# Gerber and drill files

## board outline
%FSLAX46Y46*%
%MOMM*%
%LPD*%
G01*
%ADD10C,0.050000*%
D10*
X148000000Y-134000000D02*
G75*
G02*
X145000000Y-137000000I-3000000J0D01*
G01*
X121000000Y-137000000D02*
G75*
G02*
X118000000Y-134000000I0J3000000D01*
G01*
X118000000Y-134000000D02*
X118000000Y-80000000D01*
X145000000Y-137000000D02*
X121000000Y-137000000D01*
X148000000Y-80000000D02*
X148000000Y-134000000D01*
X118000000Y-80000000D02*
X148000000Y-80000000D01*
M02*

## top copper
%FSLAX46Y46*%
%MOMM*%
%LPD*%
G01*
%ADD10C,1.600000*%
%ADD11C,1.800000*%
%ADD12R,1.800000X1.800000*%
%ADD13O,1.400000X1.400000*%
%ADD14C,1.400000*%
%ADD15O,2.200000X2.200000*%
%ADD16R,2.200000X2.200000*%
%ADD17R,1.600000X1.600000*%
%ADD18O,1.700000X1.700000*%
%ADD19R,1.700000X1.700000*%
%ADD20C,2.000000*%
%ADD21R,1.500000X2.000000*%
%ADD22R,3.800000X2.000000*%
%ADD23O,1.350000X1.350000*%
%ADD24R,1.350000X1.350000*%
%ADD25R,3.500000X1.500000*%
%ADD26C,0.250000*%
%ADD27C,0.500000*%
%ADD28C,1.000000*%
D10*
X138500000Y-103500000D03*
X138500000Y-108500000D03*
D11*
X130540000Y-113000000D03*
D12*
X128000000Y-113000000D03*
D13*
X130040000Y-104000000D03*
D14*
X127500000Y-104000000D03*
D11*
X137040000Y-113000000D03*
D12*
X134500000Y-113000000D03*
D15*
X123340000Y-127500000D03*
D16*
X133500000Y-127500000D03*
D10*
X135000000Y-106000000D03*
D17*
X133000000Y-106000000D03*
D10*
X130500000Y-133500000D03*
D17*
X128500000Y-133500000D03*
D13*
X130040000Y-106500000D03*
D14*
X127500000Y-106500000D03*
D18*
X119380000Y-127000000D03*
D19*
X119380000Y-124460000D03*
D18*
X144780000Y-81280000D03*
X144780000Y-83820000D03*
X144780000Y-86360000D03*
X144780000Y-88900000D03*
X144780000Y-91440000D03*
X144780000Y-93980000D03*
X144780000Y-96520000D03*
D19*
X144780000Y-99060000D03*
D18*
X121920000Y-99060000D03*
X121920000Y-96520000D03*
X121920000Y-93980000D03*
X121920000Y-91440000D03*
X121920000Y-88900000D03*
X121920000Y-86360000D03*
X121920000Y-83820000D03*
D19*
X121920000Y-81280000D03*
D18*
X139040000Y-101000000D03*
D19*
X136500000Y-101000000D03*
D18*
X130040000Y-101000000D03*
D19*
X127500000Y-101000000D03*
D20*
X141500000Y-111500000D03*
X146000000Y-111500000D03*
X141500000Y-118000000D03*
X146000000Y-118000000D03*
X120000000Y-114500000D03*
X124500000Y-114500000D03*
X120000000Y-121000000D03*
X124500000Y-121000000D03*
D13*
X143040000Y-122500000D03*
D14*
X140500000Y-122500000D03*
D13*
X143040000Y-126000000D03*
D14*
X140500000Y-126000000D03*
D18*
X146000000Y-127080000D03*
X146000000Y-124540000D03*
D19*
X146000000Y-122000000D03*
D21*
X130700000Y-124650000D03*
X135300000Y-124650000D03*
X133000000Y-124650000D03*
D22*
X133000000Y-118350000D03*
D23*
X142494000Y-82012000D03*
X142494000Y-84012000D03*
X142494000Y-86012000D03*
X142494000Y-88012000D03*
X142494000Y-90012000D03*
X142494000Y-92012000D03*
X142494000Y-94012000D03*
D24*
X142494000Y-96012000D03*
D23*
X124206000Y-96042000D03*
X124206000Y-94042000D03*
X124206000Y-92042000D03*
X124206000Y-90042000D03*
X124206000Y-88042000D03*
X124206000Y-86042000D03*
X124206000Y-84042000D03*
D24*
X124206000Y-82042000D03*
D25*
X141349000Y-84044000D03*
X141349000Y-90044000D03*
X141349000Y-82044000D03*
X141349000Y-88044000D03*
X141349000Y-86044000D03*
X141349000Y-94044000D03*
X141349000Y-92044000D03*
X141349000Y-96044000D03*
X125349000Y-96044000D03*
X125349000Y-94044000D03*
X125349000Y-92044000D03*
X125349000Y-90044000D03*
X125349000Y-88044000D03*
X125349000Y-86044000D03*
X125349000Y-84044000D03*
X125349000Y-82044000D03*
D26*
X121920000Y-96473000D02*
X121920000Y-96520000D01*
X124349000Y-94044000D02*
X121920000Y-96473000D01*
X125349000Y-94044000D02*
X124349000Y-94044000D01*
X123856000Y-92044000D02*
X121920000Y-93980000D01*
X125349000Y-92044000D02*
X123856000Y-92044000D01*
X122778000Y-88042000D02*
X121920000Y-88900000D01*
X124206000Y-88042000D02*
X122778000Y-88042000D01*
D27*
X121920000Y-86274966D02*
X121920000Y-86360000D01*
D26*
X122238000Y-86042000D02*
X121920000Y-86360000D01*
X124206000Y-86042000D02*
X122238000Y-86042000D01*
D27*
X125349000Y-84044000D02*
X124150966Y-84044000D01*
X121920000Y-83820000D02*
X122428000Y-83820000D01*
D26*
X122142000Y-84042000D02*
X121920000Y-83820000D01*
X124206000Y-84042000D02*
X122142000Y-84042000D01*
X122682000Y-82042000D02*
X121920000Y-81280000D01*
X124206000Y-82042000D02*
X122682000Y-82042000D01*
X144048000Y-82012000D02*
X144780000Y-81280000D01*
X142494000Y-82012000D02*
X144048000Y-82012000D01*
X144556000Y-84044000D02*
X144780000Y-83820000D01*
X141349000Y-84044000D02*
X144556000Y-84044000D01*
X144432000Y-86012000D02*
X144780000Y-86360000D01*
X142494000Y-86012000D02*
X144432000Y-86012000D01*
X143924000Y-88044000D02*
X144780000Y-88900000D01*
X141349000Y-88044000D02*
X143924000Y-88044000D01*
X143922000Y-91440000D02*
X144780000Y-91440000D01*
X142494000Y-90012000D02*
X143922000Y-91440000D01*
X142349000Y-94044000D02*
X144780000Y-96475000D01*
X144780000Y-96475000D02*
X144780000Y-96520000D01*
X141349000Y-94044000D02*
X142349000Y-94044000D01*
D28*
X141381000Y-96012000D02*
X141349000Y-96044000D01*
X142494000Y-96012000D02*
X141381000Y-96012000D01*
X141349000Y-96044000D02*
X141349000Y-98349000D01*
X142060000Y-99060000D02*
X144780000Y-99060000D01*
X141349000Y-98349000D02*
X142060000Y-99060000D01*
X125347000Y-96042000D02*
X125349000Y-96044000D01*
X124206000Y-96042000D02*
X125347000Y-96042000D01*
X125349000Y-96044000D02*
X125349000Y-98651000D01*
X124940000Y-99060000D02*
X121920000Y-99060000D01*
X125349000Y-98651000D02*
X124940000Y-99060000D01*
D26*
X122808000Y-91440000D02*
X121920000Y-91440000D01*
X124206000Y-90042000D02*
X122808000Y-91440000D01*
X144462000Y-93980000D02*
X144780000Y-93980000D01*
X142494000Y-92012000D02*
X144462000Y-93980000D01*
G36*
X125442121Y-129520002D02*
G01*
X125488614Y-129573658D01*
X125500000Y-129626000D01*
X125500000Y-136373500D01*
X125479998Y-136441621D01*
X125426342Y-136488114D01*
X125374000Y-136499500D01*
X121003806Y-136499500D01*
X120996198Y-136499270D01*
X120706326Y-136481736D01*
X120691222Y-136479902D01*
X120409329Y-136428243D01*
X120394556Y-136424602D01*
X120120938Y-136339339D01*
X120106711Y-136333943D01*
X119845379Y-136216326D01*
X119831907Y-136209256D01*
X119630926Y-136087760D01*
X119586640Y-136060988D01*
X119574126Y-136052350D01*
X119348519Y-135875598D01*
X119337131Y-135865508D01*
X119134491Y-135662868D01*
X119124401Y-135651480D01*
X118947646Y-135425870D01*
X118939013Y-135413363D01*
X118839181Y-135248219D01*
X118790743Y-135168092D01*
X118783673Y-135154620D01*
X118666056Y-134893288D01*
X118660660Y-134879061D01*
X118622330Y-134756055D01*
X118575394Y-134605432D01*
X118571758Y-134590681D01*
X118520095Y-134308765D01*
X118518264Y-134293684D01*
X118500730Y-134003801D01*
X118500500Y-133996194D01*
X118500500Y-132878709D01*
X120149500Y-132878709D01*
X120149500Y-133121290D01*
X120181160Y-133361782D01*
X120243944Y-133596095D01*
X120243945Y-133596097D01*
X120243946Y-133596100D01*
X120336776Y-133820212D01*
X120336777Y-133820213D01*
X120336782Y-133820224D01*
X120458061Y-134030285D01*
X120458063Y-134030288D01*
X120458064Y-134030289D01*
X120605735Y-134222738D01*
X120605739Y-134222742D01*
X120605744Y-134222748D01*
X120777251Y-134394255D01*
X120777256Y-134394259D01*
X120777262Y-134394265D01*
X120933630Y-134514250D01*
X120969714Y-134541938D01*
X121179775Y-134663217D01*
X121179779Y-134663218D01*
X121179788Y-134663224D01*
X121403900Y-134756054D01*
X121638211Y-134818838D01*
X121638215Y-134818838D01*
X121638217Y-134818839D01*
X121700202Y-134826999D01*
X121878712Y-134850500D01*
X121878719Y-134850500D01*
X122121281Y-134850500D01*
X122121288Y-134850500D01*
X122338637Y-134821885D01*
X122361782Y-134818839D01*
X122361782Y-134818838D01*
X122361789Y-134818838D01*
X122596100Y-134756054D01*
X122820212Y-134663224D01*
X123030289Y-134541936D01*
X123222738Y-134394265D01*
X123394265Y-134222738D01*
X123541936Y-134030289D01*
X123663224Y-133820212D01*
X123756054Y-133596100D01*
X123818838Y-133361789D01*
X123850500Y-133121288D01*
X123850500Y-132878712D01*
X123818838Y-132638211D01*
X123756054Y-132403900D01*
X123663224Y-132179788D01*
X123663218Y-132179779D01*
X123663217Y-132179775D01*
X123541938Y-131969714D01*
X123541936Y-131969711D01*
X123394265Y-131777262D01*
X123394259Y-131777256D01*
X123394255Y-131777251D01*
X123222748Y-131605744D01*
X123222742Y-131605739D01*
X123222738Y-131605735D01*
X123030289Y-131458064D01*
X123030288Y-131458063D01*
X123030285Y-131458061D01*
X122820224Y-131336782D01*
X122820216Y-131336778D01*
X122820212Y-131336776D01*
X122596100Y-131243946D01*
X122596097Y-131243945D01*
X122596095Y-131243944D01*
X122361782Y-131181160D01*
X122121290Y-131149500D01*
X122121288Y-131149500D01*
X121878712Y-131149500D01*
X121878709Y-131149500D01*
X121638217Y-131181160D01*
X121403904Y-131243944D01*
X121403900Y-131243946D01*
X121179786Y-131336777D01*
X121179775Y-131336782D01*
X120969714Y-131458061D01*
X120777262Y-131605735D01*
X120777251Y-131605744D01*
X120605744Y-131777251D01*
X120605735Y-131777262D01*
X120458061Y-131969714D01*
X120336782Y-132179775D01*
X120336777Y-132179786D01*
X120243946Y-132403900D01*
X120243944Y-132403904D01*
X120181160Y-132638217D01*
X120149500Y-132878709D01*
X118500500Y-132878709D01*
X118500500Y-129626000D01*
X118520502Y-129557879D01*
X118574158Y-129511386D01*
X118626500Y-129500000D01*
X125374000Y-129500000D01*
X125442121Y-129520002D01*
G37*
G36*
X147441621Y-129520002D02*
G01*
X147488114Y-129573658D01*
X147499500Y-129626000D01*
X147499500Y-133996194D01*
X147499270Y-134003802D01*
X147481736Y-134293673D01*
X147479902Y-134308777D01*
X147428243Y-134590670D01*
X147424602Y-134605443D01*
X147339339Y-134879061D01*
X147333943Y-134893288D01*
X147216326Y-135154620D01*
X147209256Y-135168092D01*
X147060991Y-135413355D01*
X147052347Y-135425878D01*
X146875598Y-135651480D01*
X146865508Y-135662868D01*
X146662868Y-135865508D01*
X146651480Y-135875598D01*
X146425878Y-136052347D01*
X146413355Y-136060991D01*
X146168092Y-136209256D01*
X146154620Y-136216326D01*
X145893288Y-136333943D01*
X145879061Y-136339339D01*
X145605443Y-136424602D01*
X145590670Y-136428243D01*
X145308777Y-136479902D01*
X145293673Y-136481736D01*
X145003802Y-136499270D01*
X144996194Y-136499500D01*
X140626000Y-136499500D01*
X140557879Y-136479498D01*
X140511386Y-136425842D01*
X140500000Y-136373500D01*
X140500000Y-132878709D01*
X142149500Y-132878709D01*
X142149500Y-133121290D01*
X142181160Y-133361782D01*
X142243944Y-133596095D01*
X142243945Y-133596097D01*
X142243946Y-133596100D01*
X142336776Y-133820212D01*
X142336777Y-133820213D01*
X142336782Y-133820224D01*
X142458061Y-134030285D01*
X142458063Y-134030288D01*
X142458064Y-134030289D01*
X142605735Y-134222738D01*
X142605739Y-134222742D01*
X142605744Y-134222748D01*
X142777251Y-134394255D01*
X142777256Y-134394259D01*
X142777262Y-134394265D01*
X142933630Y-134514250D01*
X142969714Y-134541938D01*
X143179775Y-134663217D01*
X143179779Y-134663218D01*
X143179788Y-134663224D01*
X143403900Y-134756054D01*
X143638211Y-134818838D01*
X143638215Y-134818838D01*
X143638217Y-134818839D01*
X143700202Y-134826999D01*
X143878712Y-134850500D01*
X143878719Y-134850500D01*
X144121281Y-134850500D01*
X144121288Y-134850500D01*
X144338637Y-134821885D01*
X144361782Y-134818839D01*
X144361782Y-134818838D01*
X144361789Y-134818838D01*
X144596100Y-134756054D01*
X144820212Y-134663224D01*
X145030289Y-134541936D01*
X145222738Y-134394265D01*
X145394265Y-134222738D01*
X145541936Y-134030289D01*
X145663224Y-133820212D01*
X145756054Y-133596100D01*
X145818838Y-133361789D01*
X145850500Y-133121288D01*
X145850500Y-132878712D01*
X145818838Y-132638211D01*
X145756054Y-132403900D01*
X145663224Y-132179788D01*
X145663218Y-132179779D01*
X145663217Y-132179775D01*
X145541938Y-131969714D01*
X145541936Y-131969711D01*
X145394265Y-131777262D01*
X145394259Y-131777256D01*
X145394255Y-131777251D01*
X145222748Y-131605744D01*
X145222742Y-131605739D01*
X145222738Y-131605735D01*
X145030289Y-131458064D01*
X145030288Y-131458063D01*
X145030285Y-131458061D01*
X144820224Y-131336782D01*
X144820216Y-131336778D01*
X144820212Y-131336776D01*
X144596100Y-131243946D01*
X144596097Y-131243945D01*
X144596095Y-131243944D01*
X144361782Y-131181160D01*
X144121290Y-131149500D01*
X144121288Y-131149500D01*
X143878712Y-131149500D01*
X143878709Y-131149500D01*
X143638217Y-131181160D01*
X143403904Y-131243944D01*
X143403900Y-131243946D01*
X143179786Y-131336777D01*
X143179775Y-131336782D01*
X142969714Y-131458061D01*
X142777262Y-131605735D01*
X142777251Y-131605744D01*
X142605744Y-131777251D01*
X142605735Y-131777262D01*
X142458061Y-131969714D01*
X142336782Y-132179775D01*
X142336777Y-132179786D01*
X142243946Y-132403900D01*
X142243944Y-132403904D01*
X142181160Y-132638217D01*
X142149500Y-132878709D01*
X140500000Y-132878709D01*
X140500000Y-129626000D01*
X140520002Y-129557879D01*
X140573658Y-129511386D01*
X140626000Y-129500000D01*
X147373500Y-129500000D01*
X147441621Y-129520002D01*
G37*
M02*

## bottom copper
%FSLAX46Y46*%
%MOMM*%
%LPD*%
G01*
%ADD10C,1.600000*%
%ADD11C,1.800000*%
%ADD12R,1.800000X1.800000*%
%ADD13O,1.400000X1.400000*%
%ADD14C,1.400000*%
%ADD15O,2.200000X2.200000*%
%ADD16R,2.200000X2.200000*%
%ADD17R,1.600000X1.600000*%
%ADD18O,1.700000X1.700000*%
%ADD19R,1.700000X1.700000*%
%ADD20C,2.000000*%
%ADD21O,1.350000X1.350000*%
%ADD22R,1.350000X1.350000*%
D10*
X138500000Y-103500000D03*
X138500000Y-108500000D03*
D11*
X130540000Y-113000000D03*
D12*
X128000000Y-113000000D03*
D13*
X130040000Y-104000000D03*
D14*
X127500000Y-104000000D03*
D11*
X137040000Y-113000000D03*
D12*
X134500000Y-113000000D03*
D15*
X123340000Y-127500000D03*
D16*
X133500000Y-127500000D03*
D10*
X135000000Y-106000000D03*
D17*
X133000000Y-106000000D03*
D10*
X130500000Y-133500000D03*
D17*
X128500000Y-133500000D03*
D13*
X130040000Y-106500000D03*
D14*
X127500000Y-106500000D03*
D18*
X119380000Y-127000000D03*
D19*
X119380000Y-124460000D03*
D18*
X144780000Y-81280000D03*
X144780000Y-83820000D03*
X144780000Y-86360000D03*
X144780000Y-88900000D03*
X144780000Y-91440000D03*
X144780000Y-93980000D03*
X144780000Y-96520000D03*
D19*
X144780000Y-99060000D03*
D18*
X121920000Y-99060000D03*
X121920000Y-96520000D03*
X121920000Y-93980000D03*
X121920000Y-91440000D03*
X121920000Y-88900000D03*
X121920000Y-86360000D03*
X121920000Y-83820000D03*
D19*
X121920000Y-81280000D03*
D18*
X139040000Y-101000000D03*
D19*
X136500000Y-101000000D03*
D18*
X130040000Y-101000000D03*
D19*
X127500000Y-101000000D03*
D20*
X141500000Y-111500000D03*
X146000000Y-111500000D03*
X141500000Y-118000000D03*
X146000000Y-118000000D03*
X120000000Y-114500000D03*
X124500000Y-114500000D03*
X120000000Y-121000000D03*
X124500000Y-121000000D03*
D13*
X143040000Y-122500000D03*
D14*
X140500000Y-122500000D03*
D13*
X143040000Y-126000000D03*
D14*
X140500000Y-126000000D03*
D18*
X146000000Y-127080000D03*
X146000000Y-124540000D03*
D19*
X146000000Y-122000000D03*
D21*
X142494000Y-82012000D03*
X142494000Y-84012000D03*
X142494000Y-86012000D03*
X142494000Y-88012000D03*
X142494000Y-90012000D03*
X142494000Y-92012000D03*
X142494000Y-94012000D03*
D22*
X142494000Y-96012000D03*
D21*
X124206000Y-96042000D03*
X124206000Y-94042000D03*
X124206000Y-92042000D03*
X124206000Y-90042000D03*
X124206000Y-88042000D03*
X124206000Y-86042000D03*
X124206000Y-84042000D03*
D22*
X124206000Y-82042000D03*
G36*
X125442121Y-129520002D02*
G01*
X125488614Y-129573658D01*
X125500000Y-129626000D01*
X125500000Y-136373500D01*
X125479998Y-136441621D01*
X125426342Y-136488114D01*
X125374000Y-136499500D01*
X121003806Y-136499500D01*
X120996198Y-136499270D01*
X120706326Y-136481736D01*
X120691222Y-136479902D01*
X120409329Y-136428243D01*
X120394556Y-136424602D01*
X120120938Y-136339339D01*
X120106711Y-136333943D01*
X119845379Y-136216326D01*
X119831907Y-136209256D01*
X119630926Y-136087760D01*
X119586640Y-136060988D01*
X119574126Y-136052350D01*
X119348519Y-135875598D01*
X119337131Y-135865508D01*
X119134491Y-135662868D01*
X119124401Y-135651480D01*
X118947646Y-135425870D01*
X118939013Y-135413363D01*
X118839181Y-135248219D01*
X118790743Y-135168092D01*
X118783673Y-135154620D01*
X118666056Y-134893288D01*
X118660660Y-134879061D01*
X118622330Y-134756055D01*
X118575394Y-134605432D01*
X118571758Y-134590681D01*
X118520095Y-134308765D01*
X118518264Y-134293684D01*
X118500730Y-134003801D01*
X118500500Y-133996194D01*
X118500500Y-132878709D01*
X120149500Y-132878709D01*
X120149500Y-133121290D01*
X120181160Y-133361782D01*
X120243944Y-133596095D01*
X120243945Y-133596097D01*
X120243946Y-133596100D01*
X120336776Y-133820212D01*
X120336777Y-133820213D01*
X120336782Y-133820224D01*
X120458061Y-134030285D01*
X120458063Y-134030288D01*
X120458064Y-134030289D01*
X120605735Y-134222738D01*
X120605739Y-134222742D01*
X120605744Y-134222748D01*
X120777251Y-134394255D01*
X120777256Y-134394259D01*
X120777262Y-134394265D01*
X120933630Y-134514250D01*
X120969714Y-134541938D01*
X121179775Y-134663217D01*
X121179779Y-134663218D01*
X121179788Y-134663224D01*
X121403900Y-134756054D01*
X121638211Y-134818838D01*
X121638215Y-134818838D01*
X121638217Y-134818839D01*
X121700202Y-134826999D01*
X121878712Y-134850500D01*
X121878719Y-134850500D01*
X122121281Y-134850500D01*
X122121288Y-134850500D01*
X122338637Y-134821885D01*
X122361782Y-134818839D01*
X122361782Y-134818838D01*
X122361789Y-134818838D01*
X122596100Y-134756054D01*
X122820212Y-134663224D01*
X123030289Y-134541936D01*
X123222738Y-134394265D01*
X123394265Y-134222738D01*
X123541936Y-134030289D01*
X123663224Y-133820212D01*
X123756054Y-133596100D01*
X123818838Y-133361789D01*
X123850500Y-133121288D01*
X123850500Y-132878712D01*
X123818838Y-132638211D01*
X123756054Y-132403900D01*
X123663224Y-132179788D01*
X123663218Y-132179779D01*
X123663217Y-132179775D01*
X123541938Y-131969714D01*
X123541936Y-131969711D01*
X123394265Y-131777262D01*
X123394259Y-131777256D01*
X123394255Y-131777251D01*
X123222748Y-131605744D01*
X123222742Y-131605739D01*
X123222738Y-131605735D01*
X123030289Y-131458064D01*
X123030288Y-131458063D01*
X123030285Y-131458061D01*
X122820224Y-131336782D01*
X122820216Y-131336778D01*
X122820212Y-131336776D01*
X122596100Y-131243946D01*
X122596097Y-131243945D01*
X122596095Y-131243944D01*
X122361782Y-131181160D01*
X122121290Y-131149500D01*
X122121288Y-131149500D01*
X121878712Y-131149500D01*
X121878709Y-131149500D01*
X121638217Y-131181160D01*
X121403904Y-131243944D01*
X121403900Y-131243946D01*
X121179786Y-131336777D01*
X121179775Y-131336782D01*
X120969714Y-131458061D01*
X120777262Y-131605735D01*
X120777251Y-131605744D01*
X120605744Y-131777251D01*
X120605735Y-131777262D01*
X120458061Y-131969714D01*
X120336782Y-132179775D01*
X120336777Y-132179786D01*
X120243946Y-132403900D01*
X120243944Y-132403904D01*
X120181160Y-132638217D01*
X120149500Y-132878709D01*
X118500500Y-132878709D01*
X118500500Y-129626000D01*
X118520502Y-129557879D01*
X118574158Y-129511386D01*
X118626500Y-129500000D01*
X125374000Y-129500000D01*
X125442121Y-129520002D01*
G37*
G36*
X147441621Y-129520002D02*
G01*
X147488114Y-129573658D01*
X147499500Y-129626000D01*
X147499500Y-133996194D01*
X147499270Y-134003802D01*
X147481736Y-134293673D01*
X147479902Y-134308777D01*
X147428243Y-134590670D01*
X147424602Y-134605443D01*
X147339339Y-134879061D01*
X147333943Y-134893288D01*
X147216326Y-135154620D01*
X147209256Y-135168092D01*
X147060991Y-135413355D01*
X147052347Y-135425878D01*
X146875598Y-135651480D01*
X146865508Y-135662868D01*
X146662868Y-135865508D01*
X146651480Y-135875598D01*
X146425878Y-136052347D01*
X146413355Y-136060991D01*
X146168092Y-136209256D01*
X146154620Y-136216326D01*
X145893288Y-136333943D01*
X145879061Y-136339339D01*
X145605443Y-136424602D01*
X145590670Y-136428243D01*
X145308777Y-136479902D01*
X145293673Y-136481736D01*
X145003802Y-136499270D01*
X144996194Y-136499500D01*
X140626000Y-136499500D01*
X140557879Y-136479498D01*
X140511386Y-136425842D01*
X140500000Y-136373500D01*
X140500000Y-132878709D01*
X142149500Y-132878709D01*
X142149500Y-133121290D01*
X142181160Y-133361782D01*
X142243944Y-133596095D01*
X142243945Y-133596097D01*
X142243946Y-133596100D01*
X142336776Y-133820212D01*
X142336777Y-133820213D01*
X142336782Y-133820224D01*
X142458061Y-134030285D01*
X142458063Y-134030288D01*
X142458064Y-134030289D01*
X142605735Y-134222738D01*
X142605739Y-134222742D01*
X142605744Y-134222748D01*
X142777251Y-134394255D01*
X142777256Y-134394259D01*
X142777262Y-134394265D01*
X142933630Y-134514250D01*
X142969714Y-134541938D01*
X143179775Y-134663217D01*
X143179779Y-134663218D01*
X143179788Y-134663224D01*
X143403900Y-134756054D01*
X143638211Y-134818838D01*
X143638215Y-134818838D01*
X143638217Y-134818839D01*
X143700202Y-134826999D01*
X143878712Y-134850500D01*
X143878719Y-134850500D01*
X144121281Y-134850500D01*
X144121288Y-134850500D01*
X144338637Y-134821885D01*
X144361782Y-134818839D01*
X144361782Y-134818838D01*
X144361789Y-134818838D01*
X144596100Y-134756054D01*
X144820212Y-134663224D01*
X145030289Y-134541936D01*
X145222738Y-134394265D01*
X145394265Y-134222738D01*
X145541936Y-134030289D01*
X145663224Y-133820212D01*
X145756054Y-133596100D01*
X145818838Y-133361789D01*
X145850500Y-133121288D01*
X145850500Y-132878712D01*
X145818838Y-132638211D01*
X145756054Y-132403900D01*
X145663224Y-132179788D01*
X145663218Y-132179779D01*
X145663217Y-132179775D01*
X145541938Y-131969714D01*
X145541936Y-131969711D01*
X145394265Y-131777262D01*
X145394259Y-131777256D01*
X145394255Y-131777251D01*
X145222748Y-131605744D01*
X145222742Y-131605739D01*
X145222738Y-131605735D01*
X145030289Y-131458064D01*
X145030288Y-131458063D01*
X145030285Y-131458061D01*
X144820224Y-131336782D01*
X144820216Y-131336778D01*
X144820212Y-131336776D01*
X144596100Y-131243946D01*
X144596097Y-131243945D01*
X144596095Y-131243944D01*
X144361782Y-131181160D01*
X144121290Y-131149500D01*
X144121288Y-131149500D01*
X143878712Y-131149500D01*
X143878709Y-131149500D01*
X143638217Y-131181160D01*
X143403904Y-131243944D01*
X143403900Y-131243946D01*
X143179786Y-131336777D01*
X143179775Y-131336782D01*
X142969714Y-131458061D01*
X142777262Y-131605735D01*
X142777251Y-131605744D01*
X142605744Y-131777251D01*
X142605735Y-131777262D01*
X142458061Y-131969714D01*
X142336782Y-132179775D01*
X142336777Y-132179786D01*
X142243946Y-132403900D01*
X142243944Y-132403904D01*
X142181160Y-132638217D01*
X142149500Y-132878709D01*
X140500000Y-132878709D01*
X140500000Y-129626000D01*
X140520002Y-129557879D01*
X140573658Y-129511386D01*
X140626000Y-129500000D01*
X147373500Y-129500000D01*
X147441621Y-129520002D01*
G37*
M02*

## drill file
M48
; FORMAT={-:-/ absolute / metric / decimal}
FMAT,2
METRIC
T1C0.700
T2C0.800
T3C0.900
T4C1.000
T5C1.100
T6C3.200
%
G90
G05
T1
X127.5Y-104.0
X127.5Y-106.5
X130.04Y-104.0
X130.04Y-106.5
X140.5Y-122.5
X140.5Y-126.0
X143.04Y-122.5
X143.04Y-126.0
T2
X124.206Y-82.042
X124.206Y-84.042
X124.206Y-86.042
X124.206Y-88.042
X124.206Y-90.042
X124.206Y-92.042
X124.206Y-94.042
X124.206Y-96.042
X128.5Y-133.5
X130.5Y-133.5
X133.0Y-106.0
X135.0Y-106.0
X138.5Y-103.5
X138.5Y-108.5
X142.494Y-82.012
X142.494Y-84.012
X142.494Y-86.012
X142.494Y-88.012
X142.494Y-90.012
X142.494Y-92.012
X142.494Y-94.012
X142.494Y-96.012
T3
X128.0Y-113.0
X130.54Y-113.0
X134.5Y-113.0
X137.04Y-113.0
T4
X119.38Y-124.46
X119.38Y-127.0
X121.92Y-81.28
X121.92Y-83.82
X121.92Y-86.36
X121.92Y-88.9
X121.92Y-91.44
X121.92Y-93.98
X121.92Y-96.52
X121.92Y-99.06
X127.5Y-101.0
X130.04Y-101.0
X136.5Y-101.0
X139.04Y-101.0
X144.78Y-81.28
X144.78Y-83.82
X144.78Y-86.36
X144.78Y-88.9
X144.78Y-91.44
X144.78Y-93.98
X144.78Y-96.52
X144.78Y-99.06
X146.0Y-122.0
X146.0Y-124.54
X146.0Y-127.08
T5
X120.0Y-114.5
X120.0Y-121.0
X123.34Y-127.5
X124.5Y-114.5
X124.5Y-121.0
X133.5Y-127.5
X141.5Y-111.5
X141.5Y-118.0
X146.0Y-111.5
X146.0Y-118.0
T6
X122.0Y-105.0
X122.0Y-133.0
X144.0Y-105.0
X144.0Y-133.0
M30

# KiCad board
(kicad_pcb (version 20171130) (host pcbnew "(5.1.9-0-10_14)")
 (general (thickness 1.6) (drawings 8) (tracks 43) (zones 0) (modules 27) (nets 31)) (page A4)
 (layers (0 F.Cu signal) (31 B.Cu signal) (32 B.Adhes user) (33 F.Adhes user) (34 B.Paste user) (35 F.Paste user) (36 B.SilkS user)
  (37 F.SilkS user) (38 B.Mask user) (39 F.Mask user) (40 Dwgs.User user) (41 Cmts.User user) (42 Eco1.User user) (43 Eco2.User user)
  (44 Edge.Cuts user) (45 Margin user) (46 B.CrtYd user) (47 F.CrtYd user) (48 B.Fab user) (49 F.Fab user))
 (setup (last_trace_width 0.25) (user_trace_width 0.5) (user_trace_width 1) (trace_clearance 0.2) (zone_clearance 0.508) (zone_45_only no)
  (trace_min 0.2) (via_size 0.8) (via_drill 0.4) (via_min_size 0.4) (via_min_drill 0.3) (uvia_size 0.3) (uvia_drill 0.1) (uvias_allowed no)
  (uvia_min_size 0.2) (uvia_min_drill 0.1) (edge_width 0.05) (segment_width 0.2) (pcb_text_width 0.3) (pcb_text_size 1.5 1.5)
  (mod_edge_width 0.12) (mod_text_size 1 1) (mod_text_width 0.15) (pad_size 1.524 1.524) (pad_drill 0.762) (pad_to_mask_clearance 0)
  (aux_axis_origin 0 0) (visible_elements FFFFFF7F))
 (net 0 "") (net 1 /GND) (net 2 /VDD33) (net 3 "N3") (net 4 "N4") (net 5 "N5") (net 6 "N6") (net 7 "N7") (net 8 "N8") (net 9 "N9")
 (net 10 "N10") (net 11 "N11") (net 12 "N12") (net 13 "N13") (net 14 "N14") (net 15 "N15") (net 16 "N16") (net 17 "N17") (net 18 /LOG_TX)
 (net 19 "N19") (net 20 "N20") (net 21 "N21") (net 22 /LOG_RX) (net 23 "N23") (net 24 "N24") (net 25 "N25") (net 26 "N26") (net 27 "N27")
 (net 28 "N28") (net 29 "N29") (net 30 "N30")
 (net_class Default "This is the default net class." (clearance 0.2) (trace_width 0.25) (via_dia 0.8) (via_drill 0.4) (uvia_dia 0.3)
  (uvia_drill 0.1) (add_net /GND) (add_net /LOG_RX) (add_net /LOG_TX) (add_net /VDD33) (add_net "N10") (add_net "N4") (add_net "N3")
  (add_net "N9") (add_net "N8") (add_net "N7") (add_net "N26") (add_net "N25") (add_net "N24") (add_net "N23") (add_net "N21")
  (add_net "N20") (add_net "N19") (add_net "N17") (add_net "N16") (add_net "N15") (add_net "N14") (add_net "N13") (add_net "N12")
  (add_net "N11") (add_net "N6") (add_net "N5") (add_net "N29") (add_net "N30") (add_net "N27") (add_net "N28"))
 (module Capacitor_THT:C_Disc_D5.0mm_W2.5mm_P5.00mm (layer F.Cu) (at 138.5 108.5 90)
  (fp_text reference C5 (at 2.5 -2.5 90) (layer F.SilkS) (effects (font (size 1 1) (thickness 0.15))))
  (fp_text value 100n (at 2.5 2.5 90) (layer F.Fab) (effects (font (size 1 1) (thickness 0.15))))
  (pad 2 thru_hole circle (at 5 0 90) (size 1.6 1.6) (drill 0.8) (layers *.Cu *.Mask) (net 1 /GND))
  (pad 1 thru_hole circle (at 0 0 90) (size 1.6 1.6) (drill 0.8) (layers *.Cu *.Mask) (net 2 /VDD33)))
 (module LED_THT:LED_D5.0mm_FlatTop (layer F.Cu) (at 128 113)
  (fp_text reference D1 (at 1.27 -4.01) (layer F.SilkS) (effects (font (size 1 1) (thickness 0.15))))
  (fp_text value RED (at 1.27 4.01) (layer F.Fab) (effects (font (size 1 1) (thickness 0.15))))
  (pad 2 thru_hole circle (at 2.54 0) (size 1.8 1.8) (drill 0.9) (layers *.Cu *.Mask) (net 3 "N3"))
  (pad 1 thru_hole rect (at 0 0) (size 1.8 1.8) (drill 0.9) (layers *.Cu *.Mask) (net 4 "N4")))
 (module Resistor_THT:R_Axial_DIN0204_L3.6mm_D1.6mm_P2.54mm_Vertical (layer F.Cu) (at 127.5 104)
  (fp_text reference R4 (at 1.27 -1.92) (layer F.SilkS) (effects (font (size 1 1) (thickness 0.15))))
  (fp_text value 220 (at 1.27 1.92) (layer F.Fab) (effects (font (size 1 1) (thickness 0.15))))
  (pad 2 thru_hole oval (at 2.54 0) (size 1.4 1.4) (drill 0.7) (layers *.Cu *.Mask) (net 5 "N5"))
  (pad 1 thru_hole circle (at 0 0) (size 1.4 1.4) (drill 0.7) (layers *.Cu *.Mask) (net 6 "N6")))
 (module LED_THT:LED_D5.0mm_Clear (layer F.Cu) (at 134.5 113)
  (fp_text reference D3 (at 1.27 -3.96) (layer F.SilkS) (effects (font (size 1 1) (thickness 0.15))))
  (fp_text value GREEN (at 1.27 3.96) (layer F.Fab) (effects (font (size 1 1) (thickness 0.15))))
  (pad 2 thru_hole circle (at 2.54 0) (size 1.8 1.8) (drill 0.9) (layers *.Cu *.Mask) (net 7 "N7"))
  (pad 1 thru_hole rect (at 0 0) (size 1.8 1.8) (drill 0.9) (layers *.Cu *.Mask) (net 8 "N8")))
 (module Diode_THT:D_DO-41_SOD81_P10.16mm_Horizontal (layer F.Cu) (at 133.5 127.5 180)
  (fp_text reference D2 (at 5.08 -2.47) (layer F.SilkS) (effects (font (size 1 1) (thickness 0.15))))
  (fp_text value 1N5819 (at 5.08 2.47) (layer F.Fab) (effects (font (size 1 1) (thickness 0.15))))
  (pad 2 thru_hole oval (at 10.16 0 180) (size 2.2 2.2) (drill 1.1) (layers *.Cu *.Mask) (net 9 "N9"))
  (pad 1 thru_hole rect (at 0 0 180) (size 2.2 2.2) (drill 1.1) (layers *.Cu *.Mask) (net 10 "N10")))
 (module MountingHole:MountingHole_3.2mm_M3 (layer F.Cu) (at 122 133)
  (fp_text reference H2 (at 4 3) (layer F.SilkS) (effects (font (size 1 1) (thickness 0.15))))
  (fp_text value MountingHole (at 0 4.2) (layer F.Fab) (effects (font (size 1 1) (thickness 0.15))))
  (pad 1 np_thru_hole circle (at 0 0) (size 3.2 3.2) (drill 3.2) (layers *.Cu *.Mask)))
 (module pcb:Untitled (layer B.Cu) (at 133 91 180)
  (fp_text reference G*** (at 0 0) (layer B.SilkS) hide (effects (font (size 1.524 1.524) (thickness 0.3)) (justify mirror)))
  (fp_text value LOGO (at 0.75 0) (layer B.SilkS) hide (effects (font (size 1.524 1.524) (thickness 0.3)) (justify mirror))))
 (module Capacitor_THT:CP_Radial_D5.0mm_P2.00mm (layer F.Cu) (at 133 106)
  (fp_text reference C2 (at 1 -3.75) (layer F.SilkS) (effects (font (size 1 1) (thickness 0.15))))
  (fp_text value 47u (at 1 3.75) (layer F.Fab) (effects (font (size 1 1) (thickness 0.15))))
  (pad 2 thru_hole circle (at 2 0) (size 1.6 1.6) (drill 0.8) (layers *.Cu *.Mask) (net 1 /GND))
  (pad 1 thru_hole rect (at 0 0) (size 1.6 1.6) (drill 0.8) (layers *.Cu *.Mask) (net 2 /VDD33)))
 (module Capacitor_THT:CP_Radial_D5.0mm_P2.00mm (layer F.Cu) (at 128.5 133.5)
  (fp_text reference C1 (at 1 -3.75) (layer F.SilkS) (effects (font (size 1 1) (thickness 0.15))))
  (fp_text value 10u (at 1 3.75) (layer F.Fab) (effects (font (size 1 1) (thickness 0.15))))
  (pad 2 thru_hole circle (at 2 0) (size 1.6 1.6) (drill 0.8) (layers *.Cu *.Mask) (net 1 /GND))
  (pad 1 thru_hole rect (at 0 0) (size 1.6 1.6) (drill 0.8) (layers *.Cu *.Mask) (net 10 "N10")))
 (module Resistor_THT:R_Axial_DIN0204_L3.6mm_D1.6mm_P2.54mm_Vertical (layer F.Cu) (at 127.5 106.5)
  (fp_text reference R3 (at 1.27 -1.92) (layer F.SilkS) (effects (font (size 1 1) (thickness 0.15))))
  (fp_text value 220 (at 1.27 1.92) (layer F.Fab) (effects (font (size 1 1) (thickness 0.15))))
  (pad 2 thru_hole oval (at 2.54 0) (size 1.4 1.4) (drill 0.7) (layers *.Cu *.Mask) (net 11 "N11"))
  (pad 1 thru_hole circle (at 0 0) (size 1.4 1.4) (drill 0.7) (layers *.Cu *.Mask) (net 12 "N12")))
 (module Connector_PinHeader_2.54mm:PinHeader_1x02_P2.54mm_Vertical (layer F.Cu) (at 119.38 124.46)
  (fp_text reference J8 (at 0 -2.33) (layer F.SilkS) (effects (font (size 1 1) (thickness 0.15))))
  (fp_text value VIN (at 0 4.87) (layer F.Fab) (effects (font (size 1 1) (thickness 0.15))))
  (pad 2 thru_hole oval (at 0 2.54) (size 1.7 1.7) (drill 1) (layers *.Cu *.Mask) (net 1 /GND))
  (pad 1 thru_hole rect (at 0 0) (size 1.7 1.7) (drill 1) (layers *.Cu *.Mask) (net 9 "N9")))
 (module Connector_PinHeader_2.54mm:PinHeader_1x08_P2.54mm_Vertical (layer F.Cu) (at 144.78 99.06 180)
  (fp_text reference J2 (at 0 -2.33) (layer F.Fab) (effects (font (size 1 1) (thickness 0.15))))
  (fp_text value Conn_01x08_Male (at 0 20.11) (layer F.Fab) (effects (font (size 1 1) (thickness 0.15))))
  (pad 8 thru_hole oval (at 0 17.78 180) (size 1.7 1.7) (drill 1) (layers *.Cu *.Mask) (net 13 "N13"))
  (pad 7 thru_hole oval (at 0 15.24 180) (size 1.7 1.7) (drill 1) (layers *.Cu *.Mask) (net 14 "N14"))
  (pad 6 thru_hole oval (at 0 12.7 180) (size 1.7 1.7) (drill 1) (layers *.Cu *.Mask) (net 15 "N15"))
  (pad 5 thru_hole oval (at 0 10.16 180) (size 1.7 1.7) (drill 1) (layers *.Cu *.Mask) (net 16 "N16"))
  (pad 4 thru_hole oval (at 0 7.62 180) (size 1.7 1.7) (drill 1) (layers *.Cu *.Mask) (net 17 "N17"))
  (pad 3 thru_hole oval (at 0 5.08 180) (size 1.7 1.7) (drill 1) (layers *.Cu *.Mask) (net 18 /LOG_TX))
  (pad 2 thru_hole oval (at 0 2.54 180) (size 1.7 1.7) (drill 1) (layers *.Cu *.Mask) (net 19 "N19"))
  (pad 1 thru_hole rect (at 0 0 180) (size 1.7 1.7) (drill 1) (layers *.Cu *.Mask) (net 1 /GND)))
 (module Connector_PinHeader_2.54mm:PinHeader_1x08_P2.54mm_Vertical (layer F.Cu) (at 121.92 81.28)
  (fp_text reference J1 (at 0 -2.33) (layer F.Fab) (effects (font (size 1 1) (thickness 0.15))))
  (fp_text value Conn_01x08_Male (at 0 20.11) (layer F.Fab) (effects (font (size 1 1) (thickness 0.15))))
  (pad 8 thru_hole oval (at 0 17.78) (size 1.7 1.7) (drill 1) (layers *.Cu *.Mask) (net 2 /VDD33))
  (pad 7 thru_hole oval (at 0 15.24) (size 1.7 1.7) (drill 1) (layers *.Cu *.Mask) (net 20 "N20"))
  (pad 6 thru_hole oval (at 0 12.7) (size 1.7 1.7) (drill 1) (layers *.Cu *.Mask) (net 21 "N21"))
  (pad 5 thru_hole oval (at 0 10.16) (size 1.7 1.7) (drill 1) (layers *.Cu *.Mask) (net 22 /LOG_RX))
  (pad 4 thru_hole oval (at 0 7.62) (size 1.7 1.7) (drill 1) (layers *.Cu *.Mask) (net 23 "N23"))
  (pad 3 thru_hole oval (at 0 5.08) (size 1.7 1.7) (drill 1) (layers *.Cu *.Mask) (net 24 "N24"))
  (pad 2 thru_hole oval (at 0 2.54) (size 1.7 1.7) (drill 1) (layers *.Cu *.Mask) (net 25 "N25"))
  (pad 1 thru_hole rect (at 0 0) (size 1.7 1.7) (drill 1) (layers *.Cu *.Mask) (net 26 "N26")))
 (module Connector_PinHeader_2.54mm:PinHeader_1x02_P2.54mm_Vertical (layer F.Cu) (at 136.5 101 90)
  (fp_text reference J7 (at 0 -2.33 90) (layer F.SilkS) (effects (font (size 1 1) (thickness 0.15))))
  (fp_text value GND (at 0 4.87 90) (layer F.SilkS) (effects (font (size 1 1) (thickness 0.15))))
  (pad 2 thru_hole oval (at 0 2.54 90) (size 1.7 1.7) (drill 1) (layers *.Cu *.Mask) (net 1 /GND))
  (pad 1 thru_hole rect (at 0 0 90) (size 1.7 1.7) (drill 1) (layers *.Cu *.Mask) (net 1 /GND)))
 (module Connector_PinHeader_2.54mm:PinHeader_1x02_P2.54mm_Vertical (layer F.Cu) (at 127.5 101 90)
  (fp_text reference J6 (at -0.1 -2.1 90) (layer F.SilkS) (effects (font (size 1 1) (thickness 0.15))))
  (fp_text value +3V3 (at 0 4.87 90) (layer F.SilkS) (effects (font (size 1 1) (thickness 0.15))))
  (pad 2 thru_hole oval (at 0 2.54 90) (size 1.7 1.7) (drill 1) (layers *.Cu *.Mask) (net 2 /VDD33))
  (pad 1 thru_hole rect (at 0 0 90) (size 1.7 1.7) (drill 1) (layers *.Cu *.Mask) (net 2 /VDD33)))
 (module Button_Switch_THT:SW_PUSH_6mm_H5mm (layer F.Cu) (at 141.5 118 90)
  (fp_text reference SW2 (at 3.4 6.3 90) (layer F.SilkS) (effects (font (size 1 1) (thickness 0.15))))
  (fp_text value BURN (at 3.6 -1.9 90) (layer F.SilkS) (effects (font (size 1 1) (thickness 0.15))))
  (pad 1 thru_hole circle (at 6.5 0 180) (size 2 2) (drill 1.1) (layers *.Cu *.Mask) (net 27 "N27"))
  (pad 2 thru_hole circle (at 6.5 4.5 180) (size 2 2) (drill 1.1) (layers *.Cu *.Mask) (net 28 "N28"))
  (pad 1 thru_hole circle (at 0 0 180) (size 2 2) (drill 1.1) (layers *.Cu *.Mask) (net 27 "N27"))
  (pad 2 thru_hole circle (at 0 4.5 180) (size 2 2) (drill 1.1) (layers *.Cu *.Mask) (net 28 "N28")))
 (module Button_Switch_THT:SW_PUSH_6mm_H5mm (layer F.Cu) (at 120 121 90)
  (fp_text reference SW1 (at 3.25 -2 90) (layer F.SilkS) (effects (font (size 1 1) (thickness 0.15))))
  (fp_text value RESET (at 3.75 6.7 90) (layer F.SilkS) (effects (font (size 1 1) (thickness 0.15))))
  (pad 1 thru_hole circle (at 6.5 0 180) (size 2 2) (drill 1.1) (layers *.Cu *.Mask) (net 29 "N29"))
  (pad 2 thru_hole circle (at 6.5 4.5 180) (size 2 2) (drill 1.1) (layers *.Cu *.Mask) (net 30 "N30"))
  (pad 1 thru_hole circle (at 0 0 180) (size 2 2) (drill 1.1) (layers *.Cu *.Mask) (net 29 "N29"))
  (pad 2 thru_hole circle (at 0 4.5 180) (size 2 2) (drill 1.1) (layers *.Cu *.Mask) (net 30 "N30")))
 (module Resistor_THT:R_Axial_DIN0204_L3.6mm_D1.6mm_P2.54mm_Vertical (layer F.Cu) (at 140.5 122.5)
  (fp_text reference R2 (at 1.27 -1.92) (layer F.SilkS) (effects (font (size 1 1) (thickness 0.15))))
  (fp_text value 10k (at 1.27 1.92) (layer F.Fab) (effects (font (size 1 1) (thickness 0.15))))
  (pad 2 thru_hole oval (at 2.54 0) (size 1.4 1.4) (drill 0.7) (layers *.Cu *.Mask) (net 18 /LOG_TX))
  (pad 1 thru_hole circle (at 0 0) (size 1.4 1.4) (drill 0.7) (layers *.Cu *.Mask) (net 2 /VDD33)))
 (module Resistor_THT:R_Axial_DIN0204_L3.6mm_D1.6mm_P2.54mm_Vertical (layer F.Cu) (at 140.5 126)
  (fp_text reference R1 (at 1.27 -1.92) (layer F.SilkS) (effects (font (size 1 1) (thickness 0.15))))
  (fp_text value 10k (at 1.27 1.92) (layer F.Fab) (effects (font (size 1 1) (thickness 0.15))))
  (pad 2 thru_hole oval (at 2.54 0) (size 1.4 1.4) (drill 0.7) (layers *.Cu *.Mask) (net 22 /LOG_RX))
  (pad 1 thru_hole circle (at 0 0) (size 1.4 1.4) (drill 0.7) (layers *.Cu *.Mask) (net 2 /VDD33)))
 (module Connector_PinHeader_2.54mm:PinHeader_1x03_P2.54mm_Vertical (layer F.Cu) (at 146 122)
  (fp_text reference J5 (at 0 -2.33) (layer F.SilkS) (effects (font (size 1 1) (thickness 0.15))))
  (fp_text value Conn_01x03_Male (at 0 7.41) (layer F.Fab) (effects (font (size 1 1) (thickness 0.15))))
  (pad 3 thru_hole oval (at 0 5.08) (size 1.7 1.7) (drill 1) (layers *.Cu *.Mask) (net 1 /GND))
  (pad 2 thru_hole oval (at 0 2.54) (size 1.7 1.7) (drill 1) (layers *.Cu *.Mask) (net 22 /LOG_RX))
  (pad 1 thru_hole rect (at 0 0) (size 1.7 1.7) (drill 1) (layers *.Cu *.Mask) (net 18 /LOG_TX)))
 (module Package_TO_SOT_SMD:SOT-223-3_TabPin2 (layer F.Cu) (at 133 121.5 90)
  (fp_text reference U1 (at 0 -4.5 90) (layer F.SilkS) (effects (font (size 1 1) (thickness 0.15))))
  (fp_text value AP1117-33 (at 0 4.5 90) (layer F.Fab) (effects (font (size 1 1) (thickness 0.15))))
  (pad 1 smd rect (at -3.15 -2.3 90) (size 2 1.5) (layers F.Cu F.Paste F.Mask) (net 1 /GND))
  (pad 3 smd rect (at -3.15 2.3 90) (size 2 1.5) (layers F.Cu F.Paste F.Mask) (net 10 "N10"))
  (pad 2 smd rect (at -3.15 0 90) (size 2 1.5) (layers F.Cu F.Paste F.Mask) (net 2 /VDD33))
  (pad 2 smd rect (at 3.15 0 90) (size 2 3.8) (layers F.Cu F.Paste F.Mask) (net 2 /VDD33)))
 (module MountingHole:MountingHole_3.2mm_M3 (layer F.Cu) (at 144 133)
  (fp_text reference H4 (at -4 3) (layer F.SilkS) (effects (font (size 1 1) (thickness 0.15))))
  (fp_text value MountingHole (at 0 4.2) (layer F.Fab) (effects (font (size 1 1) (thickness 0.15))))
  (pad 1 np_thru_hole circle (at 0 0) (size 3.2 3.2) (drill 3.2) (layers *.Cu *.Mask)))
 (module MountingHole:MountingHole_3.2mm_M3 (layer F.Cu) (at 144 105)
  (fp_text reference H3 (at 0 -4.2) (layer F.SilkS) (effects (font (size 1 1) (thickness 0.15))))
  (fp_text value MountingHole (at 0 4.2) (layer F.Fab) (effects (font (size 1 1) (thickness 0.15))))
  (pad 1 np_thru_hole circle (at 0 0) (size 3.2 3.2) (drill 3.2) (layers *.Cu *.Mask)))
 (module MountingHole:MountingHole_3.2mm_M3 (layer F.Cu) (at 122 105)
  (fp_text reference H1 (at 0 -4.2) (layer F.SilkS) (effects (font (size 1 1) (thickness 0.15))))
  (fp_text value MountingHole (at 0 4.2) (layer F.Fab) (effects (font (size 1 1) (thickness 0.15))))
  (pad 1 np_thru_hole circle (at 0 0) (size 3.2 3.2) (drill 3.2) (layers *.Cu *.Mask)))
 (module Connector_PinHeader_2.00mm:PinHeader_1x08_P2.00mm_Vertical (layer F.Cu) (at 142.494 96.012 180)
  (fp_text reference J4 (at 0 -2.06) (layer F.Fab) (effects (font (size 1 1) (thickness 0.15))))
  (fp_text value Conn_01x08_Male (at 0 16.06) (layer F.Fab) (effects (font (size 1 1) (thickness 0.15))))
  (pad 8 thru_hole oval (at 0 14 180) (size 1.35 1.35) (drill 0.8) (layers *.Cu *.Mask) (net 13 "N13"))
  (pad 7 thru_hole oval (at 0 12 180) (size 1.35 1.35) (drill 0.8) (layers *.Cu *.Mask) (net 14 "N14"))
  (pad 6 thru_hole oval (at 0 10 180) (size 1.35 1.35) (drill 0.8) (layers *.Cu *.Mask) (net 15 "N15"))
  (pad 5 thru_hole oval (at 0 8 180) (size 1.35 1.35) (drill 0.8) (layers *.Cu *.Mask) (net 16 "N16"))
  (pad 4 thru_hole oval (at 0 6 180) (size 1.35 1.35) (drill 0.8) (layers *.Cu *.Mask) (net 17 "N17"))
  (pad 3 thru_hole oval (at 0 4 180) (size 1.35 1.35) (drill 0.8) (layers *.Cu *.Mask) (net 18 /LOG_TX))
  (pad 2 thru_hole oval (at 0 2 180) (size 1.35 1.35) (drill 0.8) (layers *.Cu *.Mask) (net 19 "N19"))
  (pad 1 thru_hole rect (at 0 0 180) (size 1.35 1.35) (drill 0.8) (layers *.Cu *.Mask) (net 1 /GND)))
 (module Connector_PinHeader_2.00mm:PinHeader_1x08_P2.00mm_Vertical (layer F.Cu) (at 124.206 82.042)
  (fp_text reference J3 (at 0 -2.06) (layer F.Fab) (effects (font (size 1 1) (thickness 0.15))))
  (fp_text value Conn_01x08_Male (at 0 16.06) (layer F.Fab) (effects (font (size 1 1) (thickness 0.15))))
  (pad 8 thru_hole oval (at 0 14) (size 1.35 1.35) (drill 0.8) (layers *.Cu *.Mask) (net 2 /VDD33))
  (pad 7 thru_hole oval (at 0 12) (size 1.35 1.35) (drill 0.8) (layers *.Cu *.Mask) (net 20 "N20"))
  (pad 6 thru_hole oval (at 0 10) (size 1.35 1.35) (drill 0.8) (layers *.Cu *.Mask) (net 21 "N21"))
  (pad 5 thru_hole oval (at 0 8) (size 1.35 1.35) (drill 0.8) (layers *.Cu *.Mask) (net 22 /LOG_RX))
  (pad 4 thru_hole oval (at 0 6) (size 1.35 1.35) (drill 0.8) (layers *.Cu *.Mask) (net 23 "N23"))
  (pad 3 thru_hole oval (at 0 4) (size 1.35 1.35) (drill 0.8) (layers *.Cu *.Mask) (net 24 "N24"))
  (pad 2 thru_hole oval (at 0 2) (size 1.35 1.35) (drill 0.8) (layers *.Cu *.Mask) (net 25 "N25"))
  (pad 1 thru_hole rect (at 0 0) (size 1.35 1.35) (drill 0.8) (layers *.Cu *.Mask) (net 26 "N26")))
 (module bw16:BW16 (layer F.Cu) (at 125.349 98.044)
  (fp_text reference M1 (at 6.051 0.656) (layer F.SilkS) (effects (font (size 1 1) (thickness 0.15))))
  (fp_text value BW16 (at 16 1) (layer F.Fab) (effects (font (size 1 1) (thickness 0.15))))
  (pad 15 smd rect (at 16 -14) (size 3.5 1.5) (layers F.Cu F.Paste F.Mask) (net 14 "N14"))
  (pad 12 smd rect (at 16 -8) (size 3.5 1.5) (layers F.Cu F.Paste F.Mask) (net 17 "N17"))
  (pad 16 smd rect (at 16 -16) (size 3.5 1.5) (layers F.Cu F.Paste F.Mask) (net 13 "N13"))
  (pad 13 smd rect (at 16 -10) (size 3.5 1.5) (layers F.Cu F.Paste F.Mask) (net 16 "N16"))
  (pad 14 smd rect (at 16 -12) (size 3.5 1.5) (layers F.Cu F.Paste F.Mask) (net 15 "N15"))
  (pad 10 smd rect (at 16 -4) (size 3.5 1.5) (layers F.Cu F.Paste F.Mask) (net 19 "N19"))
  (pad 11 smd rect (at 16 -6) (size 3.5 1.5) (layers F.Cu F.Paste F.Mask) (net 18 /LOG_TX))
  (pad 9 smd rect (at 16 -2) (size 3.5 1.5) (layers F.Cu F.Paste F.Mask) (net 1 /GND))
  (pad 8 smd rect (at 0 -2) (size 3.5 1.5) (layers F.Cu F.Paste F.Mask) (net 2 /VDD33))
  (pad 7 smd rect (at 0 -4) (size 3.5 1.5) (layers F.Cu F.Paste F.Mask) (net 20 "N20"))
  (pad 6 smd rect (at 0 -6) (size 3.5 1.5) (layers F.Cu F.Paste F.Mask) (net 21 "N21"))
  (pad 5 smd rect (at 0 -8) (size 3.5 1.5) (layers F.Cu F.Paste F.Mask) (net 22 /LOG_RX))
  (pad 4 smd rect (at 0 -10) (size 3.5 1.5) (layers F.Cu F.Paste F.Mask) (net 23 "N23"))
  (pad 3 smd rect (at 0 -12) (size 3.5 1.5) (layers F.Cu F.Paste F.Mask) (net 24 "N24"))
  (pad 2 smd rect (at 0 -14) (size 3.5 1.5) (layers F.Cu F.Paste F.Mask) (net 25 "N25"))
  (pad 1 smd rect (at 0 -16) (size 3.5 1.5) (layers F.Cu F.Paste F.Mask) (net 26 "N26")))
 (gr_arc (start 145 134) (end 145 137) (angle -90) (layer Edge.Cuts) (width 0.05))
 (gr_arc (start 121 134) (end 118 134) (angle -90) (layer Edge.Cuts) (width 0.05))
 (gr_line (start 118 134) (end 118 80) (layer Edge.Cuts) (width 0.05))
 (gr_line (start 145 137) (end 121 137) (layer Edge.Cuts) (width 0.05))
 (gr_line (start 148 80) (end 148 134) (layer Edge.Cuts) (width 0.05))
 (gr_line (start 118 80) (end 148 80) (layer Edge.Cuts) (width 0.05))
 (segment (start 121.92 96.473) (end 121.92 96.52) (width 0.25) (layer F.Cu) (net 20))
 (segment (start 124.349 94.044) (end 121.92 96.473) (width 0.25) (layer F.Cu) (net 20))
 (segment (start 125.349 94.044) (end 124.349 94.044) (width 0.25) (layer F.Cu) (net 20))
 (segment (start 123.856 92.044) (end 121.92 93.98) (width 0.25) (layer F.Cu) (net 21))
 (segment (start 125.349 92.044) (end 123.856 92.044) (width 0.25) (layer F.Cu) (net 21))
 (segment (start 122.778 88.042) (end 121.92 88.9) (width 0.25) (layer F.Cu) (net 23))
 (segment (start 124.206 88.042) (end 122.778 88.042) (width 0.25) (layer F.Cu) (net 23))
 (segment (start 121.92 86.274966) (end 121.92 86.36) (width 0.5) (layer F.Cu) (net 24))
 (segment (start 122.238 86.042) (end 121.92 86.36) (width 0.25) (layer F.Cu) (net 24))
 (segment (start 124.206 86.042) (end 122.238 86.042) (width 0.25) (layer F.Cu) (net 24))
 (segment (start 125.349 84.044) (end 124.150966 84.044) (width 0.5) (layer F.Cu) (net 25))
 (segment (start 121.92 83.82) (end 122.428 83.82) (width 0.5) (layer F.Cu) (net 25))
 (segment (start 122.142 84.042) (end 121.92 83.82) (width 0.25) (layer F.Cu) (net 25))
 (segment (start 124.206 84.042) (end 122.142 84.042) (width 0.25) (layer F.Cu) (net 25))
 (segment (start 122.682 82.042) (end 121.92 81.28) (width 0.25) (layer F.Cu) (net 26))
 (segment (start 124.206 82.042) (end 122.682 82.042) (width 0.25) (layer F.Cu) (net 26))
 (segment (start 144.048 82.012) (end 144.78 81.28) (width 0.25) (layer F.Cu) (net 13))
 (segment (start 142.494 82.012) (end 144.048 82.012) (width 0.25) (layer F.Cu) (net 13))
 (segment (start 144.556 84.044) (end 144.78 83.82) (width 0.25) (layer F.Cu) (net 14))
 (segment (start 141.349 84.044) (end 144.556 84.044) (width 0.25) (layer F.Cu) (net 14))
 (segment (start 144.432 86.012) (end 144.78 86.36) (width 0.25) (layer F.Cu) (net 15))
 (segment (start 142.494 86.012) (end 144.432 86.012) (width 0.25) (layer F.Cu) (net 15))
 (segment (start 143.924 88.044) (end 144.78 88.9) (width 0.25) (layer F.Cu) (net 16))
 (segment (start 141.349 88.044) (end 143.924 88.044) (width 0.25) (layer F.Cu) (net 16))
 (segment (start 143.922 91.44) (end 144.78 91.44) (width 0.25) (layer F.Cu) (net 17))
 (segment (start 142.494 90.012) (end 143.922 91.44) (width 0.25) (layer F.Cu) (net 17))
 (segment (start 142.349 94.044) (end 144.78 96.475) (width 0.25) (layer F.Cu) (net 19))
 (segment (start 144.78 96.475) (end 144.78 96.52) (width 0.25) (layer F.Cu) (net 19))
 (segment (start 141.349 94.044) (end 142.349 94.044) (width 0.25) (layer F.Cu) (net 19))
 (segment (start 141.381 96.012) (end 141.349 96.044) (width 1) (layer F.Cu) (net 1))
 (segment (start 142.494 96.012) (end 141.381 96.012) (width 1) (layer F.Cu) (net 1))
 (segment (start 141.349 96.044) (end 141.349 98.349) (width 1) (layer F.Cu) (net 1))
 (segment (start 142.06 99.06) (end 144.78 99.06) (width 1) (layer F.Cu) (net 1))
 (segment (start 141.349 98.349) (end 142.06 99.06) (width 1) (layer F.Cu) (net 1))
 (segment (start 125.347 96.042) (end 125.349 96.044) (width 1) (layer F.Cu) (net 2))
 (segment (start 124.206 96.042) (end 125.347 96.042) (width 1) (layer F.Cu) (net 2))
 (segment (start 125.349 96.044) (end 125.349 98.651) (width 1) (layer F.Cu) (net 2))
 (segment (start 124.94 99.06) (end 121.92 99.06) (width 1) (layer F.Cu) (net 2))
 (segment (start 125.349 98.651) (end 124.94 99.06) (width 1) (layer F.Cu) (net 2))
 (segment (start 122.808 91.44) (end 121.92 91.44) (width 0.25) (layer F.Cu) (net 22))
 (segment (start 124.206 90.042) (end 122.808 91.44) (width 0.25) (layer F.Cu) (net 22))
 (segment (start 144.462 93.98) (end 144.78 93.98) (width 0.25) (layer F.Cu) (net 18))
 (segment (start 142.494 92.012) (end 144.462 93.98) (width 0.25) (layer F.Cu) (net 18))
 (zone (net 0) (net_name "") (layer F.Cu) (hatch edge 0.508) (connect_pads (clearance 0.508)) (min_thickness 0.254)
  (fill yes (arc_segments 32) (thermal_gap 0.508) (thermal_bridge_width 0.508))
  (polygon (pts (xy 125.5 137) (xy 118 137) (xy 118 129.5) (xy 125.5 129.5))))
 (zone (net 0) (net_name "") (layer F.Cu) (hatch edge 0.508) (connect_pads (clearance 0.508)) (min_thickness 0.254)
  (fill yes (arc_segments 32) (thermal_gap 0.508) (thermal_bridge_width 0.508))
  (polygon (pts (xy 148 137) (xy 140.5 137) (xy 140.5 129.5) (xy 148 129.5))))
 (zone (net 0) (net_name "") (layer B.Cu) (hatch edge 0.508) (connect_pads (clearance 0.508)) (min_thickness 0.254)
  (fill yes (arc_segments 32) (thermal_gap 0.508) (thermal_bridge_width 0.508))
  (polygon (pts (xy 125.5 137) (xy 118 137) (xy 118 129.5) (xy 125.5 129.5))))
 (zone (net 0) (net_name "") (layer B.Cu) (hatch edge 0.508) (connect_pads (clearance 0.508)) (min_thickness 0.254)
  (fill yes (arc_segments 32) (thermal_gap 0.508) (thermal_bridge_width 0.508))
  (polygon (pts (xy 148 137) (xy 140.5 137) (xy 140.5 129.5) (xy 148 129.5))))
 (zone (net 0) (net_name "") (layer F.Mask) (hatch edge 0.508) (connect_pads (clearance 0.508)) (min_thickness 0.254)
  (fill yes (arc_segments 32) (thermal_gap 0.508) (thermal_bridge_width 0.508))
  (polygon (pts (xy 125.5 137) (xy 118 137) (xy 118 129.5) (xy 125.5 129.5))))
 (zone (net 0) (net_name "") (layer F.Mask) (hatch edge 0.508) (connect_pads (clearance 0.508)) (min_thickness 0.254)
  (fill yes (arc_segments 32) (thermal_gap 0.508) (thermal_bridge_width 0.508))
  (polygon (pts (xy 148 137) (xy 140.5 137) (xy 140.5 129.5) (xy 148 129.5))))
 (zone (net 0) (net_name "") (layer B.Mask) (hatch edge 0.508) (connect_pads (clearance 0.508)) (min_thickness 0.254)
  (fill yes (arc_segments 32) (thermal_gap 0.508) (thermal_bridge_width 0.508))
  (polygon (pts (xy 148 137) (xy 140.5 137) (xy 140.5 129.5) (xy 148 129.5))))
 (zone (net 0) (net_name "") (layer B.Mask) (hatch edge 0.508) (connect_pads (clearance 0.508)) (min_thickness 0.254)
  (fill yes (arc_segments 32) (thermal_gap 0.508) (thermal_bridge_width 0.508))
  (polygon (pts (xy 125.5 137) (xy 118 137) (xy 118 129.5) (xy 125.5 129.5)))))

